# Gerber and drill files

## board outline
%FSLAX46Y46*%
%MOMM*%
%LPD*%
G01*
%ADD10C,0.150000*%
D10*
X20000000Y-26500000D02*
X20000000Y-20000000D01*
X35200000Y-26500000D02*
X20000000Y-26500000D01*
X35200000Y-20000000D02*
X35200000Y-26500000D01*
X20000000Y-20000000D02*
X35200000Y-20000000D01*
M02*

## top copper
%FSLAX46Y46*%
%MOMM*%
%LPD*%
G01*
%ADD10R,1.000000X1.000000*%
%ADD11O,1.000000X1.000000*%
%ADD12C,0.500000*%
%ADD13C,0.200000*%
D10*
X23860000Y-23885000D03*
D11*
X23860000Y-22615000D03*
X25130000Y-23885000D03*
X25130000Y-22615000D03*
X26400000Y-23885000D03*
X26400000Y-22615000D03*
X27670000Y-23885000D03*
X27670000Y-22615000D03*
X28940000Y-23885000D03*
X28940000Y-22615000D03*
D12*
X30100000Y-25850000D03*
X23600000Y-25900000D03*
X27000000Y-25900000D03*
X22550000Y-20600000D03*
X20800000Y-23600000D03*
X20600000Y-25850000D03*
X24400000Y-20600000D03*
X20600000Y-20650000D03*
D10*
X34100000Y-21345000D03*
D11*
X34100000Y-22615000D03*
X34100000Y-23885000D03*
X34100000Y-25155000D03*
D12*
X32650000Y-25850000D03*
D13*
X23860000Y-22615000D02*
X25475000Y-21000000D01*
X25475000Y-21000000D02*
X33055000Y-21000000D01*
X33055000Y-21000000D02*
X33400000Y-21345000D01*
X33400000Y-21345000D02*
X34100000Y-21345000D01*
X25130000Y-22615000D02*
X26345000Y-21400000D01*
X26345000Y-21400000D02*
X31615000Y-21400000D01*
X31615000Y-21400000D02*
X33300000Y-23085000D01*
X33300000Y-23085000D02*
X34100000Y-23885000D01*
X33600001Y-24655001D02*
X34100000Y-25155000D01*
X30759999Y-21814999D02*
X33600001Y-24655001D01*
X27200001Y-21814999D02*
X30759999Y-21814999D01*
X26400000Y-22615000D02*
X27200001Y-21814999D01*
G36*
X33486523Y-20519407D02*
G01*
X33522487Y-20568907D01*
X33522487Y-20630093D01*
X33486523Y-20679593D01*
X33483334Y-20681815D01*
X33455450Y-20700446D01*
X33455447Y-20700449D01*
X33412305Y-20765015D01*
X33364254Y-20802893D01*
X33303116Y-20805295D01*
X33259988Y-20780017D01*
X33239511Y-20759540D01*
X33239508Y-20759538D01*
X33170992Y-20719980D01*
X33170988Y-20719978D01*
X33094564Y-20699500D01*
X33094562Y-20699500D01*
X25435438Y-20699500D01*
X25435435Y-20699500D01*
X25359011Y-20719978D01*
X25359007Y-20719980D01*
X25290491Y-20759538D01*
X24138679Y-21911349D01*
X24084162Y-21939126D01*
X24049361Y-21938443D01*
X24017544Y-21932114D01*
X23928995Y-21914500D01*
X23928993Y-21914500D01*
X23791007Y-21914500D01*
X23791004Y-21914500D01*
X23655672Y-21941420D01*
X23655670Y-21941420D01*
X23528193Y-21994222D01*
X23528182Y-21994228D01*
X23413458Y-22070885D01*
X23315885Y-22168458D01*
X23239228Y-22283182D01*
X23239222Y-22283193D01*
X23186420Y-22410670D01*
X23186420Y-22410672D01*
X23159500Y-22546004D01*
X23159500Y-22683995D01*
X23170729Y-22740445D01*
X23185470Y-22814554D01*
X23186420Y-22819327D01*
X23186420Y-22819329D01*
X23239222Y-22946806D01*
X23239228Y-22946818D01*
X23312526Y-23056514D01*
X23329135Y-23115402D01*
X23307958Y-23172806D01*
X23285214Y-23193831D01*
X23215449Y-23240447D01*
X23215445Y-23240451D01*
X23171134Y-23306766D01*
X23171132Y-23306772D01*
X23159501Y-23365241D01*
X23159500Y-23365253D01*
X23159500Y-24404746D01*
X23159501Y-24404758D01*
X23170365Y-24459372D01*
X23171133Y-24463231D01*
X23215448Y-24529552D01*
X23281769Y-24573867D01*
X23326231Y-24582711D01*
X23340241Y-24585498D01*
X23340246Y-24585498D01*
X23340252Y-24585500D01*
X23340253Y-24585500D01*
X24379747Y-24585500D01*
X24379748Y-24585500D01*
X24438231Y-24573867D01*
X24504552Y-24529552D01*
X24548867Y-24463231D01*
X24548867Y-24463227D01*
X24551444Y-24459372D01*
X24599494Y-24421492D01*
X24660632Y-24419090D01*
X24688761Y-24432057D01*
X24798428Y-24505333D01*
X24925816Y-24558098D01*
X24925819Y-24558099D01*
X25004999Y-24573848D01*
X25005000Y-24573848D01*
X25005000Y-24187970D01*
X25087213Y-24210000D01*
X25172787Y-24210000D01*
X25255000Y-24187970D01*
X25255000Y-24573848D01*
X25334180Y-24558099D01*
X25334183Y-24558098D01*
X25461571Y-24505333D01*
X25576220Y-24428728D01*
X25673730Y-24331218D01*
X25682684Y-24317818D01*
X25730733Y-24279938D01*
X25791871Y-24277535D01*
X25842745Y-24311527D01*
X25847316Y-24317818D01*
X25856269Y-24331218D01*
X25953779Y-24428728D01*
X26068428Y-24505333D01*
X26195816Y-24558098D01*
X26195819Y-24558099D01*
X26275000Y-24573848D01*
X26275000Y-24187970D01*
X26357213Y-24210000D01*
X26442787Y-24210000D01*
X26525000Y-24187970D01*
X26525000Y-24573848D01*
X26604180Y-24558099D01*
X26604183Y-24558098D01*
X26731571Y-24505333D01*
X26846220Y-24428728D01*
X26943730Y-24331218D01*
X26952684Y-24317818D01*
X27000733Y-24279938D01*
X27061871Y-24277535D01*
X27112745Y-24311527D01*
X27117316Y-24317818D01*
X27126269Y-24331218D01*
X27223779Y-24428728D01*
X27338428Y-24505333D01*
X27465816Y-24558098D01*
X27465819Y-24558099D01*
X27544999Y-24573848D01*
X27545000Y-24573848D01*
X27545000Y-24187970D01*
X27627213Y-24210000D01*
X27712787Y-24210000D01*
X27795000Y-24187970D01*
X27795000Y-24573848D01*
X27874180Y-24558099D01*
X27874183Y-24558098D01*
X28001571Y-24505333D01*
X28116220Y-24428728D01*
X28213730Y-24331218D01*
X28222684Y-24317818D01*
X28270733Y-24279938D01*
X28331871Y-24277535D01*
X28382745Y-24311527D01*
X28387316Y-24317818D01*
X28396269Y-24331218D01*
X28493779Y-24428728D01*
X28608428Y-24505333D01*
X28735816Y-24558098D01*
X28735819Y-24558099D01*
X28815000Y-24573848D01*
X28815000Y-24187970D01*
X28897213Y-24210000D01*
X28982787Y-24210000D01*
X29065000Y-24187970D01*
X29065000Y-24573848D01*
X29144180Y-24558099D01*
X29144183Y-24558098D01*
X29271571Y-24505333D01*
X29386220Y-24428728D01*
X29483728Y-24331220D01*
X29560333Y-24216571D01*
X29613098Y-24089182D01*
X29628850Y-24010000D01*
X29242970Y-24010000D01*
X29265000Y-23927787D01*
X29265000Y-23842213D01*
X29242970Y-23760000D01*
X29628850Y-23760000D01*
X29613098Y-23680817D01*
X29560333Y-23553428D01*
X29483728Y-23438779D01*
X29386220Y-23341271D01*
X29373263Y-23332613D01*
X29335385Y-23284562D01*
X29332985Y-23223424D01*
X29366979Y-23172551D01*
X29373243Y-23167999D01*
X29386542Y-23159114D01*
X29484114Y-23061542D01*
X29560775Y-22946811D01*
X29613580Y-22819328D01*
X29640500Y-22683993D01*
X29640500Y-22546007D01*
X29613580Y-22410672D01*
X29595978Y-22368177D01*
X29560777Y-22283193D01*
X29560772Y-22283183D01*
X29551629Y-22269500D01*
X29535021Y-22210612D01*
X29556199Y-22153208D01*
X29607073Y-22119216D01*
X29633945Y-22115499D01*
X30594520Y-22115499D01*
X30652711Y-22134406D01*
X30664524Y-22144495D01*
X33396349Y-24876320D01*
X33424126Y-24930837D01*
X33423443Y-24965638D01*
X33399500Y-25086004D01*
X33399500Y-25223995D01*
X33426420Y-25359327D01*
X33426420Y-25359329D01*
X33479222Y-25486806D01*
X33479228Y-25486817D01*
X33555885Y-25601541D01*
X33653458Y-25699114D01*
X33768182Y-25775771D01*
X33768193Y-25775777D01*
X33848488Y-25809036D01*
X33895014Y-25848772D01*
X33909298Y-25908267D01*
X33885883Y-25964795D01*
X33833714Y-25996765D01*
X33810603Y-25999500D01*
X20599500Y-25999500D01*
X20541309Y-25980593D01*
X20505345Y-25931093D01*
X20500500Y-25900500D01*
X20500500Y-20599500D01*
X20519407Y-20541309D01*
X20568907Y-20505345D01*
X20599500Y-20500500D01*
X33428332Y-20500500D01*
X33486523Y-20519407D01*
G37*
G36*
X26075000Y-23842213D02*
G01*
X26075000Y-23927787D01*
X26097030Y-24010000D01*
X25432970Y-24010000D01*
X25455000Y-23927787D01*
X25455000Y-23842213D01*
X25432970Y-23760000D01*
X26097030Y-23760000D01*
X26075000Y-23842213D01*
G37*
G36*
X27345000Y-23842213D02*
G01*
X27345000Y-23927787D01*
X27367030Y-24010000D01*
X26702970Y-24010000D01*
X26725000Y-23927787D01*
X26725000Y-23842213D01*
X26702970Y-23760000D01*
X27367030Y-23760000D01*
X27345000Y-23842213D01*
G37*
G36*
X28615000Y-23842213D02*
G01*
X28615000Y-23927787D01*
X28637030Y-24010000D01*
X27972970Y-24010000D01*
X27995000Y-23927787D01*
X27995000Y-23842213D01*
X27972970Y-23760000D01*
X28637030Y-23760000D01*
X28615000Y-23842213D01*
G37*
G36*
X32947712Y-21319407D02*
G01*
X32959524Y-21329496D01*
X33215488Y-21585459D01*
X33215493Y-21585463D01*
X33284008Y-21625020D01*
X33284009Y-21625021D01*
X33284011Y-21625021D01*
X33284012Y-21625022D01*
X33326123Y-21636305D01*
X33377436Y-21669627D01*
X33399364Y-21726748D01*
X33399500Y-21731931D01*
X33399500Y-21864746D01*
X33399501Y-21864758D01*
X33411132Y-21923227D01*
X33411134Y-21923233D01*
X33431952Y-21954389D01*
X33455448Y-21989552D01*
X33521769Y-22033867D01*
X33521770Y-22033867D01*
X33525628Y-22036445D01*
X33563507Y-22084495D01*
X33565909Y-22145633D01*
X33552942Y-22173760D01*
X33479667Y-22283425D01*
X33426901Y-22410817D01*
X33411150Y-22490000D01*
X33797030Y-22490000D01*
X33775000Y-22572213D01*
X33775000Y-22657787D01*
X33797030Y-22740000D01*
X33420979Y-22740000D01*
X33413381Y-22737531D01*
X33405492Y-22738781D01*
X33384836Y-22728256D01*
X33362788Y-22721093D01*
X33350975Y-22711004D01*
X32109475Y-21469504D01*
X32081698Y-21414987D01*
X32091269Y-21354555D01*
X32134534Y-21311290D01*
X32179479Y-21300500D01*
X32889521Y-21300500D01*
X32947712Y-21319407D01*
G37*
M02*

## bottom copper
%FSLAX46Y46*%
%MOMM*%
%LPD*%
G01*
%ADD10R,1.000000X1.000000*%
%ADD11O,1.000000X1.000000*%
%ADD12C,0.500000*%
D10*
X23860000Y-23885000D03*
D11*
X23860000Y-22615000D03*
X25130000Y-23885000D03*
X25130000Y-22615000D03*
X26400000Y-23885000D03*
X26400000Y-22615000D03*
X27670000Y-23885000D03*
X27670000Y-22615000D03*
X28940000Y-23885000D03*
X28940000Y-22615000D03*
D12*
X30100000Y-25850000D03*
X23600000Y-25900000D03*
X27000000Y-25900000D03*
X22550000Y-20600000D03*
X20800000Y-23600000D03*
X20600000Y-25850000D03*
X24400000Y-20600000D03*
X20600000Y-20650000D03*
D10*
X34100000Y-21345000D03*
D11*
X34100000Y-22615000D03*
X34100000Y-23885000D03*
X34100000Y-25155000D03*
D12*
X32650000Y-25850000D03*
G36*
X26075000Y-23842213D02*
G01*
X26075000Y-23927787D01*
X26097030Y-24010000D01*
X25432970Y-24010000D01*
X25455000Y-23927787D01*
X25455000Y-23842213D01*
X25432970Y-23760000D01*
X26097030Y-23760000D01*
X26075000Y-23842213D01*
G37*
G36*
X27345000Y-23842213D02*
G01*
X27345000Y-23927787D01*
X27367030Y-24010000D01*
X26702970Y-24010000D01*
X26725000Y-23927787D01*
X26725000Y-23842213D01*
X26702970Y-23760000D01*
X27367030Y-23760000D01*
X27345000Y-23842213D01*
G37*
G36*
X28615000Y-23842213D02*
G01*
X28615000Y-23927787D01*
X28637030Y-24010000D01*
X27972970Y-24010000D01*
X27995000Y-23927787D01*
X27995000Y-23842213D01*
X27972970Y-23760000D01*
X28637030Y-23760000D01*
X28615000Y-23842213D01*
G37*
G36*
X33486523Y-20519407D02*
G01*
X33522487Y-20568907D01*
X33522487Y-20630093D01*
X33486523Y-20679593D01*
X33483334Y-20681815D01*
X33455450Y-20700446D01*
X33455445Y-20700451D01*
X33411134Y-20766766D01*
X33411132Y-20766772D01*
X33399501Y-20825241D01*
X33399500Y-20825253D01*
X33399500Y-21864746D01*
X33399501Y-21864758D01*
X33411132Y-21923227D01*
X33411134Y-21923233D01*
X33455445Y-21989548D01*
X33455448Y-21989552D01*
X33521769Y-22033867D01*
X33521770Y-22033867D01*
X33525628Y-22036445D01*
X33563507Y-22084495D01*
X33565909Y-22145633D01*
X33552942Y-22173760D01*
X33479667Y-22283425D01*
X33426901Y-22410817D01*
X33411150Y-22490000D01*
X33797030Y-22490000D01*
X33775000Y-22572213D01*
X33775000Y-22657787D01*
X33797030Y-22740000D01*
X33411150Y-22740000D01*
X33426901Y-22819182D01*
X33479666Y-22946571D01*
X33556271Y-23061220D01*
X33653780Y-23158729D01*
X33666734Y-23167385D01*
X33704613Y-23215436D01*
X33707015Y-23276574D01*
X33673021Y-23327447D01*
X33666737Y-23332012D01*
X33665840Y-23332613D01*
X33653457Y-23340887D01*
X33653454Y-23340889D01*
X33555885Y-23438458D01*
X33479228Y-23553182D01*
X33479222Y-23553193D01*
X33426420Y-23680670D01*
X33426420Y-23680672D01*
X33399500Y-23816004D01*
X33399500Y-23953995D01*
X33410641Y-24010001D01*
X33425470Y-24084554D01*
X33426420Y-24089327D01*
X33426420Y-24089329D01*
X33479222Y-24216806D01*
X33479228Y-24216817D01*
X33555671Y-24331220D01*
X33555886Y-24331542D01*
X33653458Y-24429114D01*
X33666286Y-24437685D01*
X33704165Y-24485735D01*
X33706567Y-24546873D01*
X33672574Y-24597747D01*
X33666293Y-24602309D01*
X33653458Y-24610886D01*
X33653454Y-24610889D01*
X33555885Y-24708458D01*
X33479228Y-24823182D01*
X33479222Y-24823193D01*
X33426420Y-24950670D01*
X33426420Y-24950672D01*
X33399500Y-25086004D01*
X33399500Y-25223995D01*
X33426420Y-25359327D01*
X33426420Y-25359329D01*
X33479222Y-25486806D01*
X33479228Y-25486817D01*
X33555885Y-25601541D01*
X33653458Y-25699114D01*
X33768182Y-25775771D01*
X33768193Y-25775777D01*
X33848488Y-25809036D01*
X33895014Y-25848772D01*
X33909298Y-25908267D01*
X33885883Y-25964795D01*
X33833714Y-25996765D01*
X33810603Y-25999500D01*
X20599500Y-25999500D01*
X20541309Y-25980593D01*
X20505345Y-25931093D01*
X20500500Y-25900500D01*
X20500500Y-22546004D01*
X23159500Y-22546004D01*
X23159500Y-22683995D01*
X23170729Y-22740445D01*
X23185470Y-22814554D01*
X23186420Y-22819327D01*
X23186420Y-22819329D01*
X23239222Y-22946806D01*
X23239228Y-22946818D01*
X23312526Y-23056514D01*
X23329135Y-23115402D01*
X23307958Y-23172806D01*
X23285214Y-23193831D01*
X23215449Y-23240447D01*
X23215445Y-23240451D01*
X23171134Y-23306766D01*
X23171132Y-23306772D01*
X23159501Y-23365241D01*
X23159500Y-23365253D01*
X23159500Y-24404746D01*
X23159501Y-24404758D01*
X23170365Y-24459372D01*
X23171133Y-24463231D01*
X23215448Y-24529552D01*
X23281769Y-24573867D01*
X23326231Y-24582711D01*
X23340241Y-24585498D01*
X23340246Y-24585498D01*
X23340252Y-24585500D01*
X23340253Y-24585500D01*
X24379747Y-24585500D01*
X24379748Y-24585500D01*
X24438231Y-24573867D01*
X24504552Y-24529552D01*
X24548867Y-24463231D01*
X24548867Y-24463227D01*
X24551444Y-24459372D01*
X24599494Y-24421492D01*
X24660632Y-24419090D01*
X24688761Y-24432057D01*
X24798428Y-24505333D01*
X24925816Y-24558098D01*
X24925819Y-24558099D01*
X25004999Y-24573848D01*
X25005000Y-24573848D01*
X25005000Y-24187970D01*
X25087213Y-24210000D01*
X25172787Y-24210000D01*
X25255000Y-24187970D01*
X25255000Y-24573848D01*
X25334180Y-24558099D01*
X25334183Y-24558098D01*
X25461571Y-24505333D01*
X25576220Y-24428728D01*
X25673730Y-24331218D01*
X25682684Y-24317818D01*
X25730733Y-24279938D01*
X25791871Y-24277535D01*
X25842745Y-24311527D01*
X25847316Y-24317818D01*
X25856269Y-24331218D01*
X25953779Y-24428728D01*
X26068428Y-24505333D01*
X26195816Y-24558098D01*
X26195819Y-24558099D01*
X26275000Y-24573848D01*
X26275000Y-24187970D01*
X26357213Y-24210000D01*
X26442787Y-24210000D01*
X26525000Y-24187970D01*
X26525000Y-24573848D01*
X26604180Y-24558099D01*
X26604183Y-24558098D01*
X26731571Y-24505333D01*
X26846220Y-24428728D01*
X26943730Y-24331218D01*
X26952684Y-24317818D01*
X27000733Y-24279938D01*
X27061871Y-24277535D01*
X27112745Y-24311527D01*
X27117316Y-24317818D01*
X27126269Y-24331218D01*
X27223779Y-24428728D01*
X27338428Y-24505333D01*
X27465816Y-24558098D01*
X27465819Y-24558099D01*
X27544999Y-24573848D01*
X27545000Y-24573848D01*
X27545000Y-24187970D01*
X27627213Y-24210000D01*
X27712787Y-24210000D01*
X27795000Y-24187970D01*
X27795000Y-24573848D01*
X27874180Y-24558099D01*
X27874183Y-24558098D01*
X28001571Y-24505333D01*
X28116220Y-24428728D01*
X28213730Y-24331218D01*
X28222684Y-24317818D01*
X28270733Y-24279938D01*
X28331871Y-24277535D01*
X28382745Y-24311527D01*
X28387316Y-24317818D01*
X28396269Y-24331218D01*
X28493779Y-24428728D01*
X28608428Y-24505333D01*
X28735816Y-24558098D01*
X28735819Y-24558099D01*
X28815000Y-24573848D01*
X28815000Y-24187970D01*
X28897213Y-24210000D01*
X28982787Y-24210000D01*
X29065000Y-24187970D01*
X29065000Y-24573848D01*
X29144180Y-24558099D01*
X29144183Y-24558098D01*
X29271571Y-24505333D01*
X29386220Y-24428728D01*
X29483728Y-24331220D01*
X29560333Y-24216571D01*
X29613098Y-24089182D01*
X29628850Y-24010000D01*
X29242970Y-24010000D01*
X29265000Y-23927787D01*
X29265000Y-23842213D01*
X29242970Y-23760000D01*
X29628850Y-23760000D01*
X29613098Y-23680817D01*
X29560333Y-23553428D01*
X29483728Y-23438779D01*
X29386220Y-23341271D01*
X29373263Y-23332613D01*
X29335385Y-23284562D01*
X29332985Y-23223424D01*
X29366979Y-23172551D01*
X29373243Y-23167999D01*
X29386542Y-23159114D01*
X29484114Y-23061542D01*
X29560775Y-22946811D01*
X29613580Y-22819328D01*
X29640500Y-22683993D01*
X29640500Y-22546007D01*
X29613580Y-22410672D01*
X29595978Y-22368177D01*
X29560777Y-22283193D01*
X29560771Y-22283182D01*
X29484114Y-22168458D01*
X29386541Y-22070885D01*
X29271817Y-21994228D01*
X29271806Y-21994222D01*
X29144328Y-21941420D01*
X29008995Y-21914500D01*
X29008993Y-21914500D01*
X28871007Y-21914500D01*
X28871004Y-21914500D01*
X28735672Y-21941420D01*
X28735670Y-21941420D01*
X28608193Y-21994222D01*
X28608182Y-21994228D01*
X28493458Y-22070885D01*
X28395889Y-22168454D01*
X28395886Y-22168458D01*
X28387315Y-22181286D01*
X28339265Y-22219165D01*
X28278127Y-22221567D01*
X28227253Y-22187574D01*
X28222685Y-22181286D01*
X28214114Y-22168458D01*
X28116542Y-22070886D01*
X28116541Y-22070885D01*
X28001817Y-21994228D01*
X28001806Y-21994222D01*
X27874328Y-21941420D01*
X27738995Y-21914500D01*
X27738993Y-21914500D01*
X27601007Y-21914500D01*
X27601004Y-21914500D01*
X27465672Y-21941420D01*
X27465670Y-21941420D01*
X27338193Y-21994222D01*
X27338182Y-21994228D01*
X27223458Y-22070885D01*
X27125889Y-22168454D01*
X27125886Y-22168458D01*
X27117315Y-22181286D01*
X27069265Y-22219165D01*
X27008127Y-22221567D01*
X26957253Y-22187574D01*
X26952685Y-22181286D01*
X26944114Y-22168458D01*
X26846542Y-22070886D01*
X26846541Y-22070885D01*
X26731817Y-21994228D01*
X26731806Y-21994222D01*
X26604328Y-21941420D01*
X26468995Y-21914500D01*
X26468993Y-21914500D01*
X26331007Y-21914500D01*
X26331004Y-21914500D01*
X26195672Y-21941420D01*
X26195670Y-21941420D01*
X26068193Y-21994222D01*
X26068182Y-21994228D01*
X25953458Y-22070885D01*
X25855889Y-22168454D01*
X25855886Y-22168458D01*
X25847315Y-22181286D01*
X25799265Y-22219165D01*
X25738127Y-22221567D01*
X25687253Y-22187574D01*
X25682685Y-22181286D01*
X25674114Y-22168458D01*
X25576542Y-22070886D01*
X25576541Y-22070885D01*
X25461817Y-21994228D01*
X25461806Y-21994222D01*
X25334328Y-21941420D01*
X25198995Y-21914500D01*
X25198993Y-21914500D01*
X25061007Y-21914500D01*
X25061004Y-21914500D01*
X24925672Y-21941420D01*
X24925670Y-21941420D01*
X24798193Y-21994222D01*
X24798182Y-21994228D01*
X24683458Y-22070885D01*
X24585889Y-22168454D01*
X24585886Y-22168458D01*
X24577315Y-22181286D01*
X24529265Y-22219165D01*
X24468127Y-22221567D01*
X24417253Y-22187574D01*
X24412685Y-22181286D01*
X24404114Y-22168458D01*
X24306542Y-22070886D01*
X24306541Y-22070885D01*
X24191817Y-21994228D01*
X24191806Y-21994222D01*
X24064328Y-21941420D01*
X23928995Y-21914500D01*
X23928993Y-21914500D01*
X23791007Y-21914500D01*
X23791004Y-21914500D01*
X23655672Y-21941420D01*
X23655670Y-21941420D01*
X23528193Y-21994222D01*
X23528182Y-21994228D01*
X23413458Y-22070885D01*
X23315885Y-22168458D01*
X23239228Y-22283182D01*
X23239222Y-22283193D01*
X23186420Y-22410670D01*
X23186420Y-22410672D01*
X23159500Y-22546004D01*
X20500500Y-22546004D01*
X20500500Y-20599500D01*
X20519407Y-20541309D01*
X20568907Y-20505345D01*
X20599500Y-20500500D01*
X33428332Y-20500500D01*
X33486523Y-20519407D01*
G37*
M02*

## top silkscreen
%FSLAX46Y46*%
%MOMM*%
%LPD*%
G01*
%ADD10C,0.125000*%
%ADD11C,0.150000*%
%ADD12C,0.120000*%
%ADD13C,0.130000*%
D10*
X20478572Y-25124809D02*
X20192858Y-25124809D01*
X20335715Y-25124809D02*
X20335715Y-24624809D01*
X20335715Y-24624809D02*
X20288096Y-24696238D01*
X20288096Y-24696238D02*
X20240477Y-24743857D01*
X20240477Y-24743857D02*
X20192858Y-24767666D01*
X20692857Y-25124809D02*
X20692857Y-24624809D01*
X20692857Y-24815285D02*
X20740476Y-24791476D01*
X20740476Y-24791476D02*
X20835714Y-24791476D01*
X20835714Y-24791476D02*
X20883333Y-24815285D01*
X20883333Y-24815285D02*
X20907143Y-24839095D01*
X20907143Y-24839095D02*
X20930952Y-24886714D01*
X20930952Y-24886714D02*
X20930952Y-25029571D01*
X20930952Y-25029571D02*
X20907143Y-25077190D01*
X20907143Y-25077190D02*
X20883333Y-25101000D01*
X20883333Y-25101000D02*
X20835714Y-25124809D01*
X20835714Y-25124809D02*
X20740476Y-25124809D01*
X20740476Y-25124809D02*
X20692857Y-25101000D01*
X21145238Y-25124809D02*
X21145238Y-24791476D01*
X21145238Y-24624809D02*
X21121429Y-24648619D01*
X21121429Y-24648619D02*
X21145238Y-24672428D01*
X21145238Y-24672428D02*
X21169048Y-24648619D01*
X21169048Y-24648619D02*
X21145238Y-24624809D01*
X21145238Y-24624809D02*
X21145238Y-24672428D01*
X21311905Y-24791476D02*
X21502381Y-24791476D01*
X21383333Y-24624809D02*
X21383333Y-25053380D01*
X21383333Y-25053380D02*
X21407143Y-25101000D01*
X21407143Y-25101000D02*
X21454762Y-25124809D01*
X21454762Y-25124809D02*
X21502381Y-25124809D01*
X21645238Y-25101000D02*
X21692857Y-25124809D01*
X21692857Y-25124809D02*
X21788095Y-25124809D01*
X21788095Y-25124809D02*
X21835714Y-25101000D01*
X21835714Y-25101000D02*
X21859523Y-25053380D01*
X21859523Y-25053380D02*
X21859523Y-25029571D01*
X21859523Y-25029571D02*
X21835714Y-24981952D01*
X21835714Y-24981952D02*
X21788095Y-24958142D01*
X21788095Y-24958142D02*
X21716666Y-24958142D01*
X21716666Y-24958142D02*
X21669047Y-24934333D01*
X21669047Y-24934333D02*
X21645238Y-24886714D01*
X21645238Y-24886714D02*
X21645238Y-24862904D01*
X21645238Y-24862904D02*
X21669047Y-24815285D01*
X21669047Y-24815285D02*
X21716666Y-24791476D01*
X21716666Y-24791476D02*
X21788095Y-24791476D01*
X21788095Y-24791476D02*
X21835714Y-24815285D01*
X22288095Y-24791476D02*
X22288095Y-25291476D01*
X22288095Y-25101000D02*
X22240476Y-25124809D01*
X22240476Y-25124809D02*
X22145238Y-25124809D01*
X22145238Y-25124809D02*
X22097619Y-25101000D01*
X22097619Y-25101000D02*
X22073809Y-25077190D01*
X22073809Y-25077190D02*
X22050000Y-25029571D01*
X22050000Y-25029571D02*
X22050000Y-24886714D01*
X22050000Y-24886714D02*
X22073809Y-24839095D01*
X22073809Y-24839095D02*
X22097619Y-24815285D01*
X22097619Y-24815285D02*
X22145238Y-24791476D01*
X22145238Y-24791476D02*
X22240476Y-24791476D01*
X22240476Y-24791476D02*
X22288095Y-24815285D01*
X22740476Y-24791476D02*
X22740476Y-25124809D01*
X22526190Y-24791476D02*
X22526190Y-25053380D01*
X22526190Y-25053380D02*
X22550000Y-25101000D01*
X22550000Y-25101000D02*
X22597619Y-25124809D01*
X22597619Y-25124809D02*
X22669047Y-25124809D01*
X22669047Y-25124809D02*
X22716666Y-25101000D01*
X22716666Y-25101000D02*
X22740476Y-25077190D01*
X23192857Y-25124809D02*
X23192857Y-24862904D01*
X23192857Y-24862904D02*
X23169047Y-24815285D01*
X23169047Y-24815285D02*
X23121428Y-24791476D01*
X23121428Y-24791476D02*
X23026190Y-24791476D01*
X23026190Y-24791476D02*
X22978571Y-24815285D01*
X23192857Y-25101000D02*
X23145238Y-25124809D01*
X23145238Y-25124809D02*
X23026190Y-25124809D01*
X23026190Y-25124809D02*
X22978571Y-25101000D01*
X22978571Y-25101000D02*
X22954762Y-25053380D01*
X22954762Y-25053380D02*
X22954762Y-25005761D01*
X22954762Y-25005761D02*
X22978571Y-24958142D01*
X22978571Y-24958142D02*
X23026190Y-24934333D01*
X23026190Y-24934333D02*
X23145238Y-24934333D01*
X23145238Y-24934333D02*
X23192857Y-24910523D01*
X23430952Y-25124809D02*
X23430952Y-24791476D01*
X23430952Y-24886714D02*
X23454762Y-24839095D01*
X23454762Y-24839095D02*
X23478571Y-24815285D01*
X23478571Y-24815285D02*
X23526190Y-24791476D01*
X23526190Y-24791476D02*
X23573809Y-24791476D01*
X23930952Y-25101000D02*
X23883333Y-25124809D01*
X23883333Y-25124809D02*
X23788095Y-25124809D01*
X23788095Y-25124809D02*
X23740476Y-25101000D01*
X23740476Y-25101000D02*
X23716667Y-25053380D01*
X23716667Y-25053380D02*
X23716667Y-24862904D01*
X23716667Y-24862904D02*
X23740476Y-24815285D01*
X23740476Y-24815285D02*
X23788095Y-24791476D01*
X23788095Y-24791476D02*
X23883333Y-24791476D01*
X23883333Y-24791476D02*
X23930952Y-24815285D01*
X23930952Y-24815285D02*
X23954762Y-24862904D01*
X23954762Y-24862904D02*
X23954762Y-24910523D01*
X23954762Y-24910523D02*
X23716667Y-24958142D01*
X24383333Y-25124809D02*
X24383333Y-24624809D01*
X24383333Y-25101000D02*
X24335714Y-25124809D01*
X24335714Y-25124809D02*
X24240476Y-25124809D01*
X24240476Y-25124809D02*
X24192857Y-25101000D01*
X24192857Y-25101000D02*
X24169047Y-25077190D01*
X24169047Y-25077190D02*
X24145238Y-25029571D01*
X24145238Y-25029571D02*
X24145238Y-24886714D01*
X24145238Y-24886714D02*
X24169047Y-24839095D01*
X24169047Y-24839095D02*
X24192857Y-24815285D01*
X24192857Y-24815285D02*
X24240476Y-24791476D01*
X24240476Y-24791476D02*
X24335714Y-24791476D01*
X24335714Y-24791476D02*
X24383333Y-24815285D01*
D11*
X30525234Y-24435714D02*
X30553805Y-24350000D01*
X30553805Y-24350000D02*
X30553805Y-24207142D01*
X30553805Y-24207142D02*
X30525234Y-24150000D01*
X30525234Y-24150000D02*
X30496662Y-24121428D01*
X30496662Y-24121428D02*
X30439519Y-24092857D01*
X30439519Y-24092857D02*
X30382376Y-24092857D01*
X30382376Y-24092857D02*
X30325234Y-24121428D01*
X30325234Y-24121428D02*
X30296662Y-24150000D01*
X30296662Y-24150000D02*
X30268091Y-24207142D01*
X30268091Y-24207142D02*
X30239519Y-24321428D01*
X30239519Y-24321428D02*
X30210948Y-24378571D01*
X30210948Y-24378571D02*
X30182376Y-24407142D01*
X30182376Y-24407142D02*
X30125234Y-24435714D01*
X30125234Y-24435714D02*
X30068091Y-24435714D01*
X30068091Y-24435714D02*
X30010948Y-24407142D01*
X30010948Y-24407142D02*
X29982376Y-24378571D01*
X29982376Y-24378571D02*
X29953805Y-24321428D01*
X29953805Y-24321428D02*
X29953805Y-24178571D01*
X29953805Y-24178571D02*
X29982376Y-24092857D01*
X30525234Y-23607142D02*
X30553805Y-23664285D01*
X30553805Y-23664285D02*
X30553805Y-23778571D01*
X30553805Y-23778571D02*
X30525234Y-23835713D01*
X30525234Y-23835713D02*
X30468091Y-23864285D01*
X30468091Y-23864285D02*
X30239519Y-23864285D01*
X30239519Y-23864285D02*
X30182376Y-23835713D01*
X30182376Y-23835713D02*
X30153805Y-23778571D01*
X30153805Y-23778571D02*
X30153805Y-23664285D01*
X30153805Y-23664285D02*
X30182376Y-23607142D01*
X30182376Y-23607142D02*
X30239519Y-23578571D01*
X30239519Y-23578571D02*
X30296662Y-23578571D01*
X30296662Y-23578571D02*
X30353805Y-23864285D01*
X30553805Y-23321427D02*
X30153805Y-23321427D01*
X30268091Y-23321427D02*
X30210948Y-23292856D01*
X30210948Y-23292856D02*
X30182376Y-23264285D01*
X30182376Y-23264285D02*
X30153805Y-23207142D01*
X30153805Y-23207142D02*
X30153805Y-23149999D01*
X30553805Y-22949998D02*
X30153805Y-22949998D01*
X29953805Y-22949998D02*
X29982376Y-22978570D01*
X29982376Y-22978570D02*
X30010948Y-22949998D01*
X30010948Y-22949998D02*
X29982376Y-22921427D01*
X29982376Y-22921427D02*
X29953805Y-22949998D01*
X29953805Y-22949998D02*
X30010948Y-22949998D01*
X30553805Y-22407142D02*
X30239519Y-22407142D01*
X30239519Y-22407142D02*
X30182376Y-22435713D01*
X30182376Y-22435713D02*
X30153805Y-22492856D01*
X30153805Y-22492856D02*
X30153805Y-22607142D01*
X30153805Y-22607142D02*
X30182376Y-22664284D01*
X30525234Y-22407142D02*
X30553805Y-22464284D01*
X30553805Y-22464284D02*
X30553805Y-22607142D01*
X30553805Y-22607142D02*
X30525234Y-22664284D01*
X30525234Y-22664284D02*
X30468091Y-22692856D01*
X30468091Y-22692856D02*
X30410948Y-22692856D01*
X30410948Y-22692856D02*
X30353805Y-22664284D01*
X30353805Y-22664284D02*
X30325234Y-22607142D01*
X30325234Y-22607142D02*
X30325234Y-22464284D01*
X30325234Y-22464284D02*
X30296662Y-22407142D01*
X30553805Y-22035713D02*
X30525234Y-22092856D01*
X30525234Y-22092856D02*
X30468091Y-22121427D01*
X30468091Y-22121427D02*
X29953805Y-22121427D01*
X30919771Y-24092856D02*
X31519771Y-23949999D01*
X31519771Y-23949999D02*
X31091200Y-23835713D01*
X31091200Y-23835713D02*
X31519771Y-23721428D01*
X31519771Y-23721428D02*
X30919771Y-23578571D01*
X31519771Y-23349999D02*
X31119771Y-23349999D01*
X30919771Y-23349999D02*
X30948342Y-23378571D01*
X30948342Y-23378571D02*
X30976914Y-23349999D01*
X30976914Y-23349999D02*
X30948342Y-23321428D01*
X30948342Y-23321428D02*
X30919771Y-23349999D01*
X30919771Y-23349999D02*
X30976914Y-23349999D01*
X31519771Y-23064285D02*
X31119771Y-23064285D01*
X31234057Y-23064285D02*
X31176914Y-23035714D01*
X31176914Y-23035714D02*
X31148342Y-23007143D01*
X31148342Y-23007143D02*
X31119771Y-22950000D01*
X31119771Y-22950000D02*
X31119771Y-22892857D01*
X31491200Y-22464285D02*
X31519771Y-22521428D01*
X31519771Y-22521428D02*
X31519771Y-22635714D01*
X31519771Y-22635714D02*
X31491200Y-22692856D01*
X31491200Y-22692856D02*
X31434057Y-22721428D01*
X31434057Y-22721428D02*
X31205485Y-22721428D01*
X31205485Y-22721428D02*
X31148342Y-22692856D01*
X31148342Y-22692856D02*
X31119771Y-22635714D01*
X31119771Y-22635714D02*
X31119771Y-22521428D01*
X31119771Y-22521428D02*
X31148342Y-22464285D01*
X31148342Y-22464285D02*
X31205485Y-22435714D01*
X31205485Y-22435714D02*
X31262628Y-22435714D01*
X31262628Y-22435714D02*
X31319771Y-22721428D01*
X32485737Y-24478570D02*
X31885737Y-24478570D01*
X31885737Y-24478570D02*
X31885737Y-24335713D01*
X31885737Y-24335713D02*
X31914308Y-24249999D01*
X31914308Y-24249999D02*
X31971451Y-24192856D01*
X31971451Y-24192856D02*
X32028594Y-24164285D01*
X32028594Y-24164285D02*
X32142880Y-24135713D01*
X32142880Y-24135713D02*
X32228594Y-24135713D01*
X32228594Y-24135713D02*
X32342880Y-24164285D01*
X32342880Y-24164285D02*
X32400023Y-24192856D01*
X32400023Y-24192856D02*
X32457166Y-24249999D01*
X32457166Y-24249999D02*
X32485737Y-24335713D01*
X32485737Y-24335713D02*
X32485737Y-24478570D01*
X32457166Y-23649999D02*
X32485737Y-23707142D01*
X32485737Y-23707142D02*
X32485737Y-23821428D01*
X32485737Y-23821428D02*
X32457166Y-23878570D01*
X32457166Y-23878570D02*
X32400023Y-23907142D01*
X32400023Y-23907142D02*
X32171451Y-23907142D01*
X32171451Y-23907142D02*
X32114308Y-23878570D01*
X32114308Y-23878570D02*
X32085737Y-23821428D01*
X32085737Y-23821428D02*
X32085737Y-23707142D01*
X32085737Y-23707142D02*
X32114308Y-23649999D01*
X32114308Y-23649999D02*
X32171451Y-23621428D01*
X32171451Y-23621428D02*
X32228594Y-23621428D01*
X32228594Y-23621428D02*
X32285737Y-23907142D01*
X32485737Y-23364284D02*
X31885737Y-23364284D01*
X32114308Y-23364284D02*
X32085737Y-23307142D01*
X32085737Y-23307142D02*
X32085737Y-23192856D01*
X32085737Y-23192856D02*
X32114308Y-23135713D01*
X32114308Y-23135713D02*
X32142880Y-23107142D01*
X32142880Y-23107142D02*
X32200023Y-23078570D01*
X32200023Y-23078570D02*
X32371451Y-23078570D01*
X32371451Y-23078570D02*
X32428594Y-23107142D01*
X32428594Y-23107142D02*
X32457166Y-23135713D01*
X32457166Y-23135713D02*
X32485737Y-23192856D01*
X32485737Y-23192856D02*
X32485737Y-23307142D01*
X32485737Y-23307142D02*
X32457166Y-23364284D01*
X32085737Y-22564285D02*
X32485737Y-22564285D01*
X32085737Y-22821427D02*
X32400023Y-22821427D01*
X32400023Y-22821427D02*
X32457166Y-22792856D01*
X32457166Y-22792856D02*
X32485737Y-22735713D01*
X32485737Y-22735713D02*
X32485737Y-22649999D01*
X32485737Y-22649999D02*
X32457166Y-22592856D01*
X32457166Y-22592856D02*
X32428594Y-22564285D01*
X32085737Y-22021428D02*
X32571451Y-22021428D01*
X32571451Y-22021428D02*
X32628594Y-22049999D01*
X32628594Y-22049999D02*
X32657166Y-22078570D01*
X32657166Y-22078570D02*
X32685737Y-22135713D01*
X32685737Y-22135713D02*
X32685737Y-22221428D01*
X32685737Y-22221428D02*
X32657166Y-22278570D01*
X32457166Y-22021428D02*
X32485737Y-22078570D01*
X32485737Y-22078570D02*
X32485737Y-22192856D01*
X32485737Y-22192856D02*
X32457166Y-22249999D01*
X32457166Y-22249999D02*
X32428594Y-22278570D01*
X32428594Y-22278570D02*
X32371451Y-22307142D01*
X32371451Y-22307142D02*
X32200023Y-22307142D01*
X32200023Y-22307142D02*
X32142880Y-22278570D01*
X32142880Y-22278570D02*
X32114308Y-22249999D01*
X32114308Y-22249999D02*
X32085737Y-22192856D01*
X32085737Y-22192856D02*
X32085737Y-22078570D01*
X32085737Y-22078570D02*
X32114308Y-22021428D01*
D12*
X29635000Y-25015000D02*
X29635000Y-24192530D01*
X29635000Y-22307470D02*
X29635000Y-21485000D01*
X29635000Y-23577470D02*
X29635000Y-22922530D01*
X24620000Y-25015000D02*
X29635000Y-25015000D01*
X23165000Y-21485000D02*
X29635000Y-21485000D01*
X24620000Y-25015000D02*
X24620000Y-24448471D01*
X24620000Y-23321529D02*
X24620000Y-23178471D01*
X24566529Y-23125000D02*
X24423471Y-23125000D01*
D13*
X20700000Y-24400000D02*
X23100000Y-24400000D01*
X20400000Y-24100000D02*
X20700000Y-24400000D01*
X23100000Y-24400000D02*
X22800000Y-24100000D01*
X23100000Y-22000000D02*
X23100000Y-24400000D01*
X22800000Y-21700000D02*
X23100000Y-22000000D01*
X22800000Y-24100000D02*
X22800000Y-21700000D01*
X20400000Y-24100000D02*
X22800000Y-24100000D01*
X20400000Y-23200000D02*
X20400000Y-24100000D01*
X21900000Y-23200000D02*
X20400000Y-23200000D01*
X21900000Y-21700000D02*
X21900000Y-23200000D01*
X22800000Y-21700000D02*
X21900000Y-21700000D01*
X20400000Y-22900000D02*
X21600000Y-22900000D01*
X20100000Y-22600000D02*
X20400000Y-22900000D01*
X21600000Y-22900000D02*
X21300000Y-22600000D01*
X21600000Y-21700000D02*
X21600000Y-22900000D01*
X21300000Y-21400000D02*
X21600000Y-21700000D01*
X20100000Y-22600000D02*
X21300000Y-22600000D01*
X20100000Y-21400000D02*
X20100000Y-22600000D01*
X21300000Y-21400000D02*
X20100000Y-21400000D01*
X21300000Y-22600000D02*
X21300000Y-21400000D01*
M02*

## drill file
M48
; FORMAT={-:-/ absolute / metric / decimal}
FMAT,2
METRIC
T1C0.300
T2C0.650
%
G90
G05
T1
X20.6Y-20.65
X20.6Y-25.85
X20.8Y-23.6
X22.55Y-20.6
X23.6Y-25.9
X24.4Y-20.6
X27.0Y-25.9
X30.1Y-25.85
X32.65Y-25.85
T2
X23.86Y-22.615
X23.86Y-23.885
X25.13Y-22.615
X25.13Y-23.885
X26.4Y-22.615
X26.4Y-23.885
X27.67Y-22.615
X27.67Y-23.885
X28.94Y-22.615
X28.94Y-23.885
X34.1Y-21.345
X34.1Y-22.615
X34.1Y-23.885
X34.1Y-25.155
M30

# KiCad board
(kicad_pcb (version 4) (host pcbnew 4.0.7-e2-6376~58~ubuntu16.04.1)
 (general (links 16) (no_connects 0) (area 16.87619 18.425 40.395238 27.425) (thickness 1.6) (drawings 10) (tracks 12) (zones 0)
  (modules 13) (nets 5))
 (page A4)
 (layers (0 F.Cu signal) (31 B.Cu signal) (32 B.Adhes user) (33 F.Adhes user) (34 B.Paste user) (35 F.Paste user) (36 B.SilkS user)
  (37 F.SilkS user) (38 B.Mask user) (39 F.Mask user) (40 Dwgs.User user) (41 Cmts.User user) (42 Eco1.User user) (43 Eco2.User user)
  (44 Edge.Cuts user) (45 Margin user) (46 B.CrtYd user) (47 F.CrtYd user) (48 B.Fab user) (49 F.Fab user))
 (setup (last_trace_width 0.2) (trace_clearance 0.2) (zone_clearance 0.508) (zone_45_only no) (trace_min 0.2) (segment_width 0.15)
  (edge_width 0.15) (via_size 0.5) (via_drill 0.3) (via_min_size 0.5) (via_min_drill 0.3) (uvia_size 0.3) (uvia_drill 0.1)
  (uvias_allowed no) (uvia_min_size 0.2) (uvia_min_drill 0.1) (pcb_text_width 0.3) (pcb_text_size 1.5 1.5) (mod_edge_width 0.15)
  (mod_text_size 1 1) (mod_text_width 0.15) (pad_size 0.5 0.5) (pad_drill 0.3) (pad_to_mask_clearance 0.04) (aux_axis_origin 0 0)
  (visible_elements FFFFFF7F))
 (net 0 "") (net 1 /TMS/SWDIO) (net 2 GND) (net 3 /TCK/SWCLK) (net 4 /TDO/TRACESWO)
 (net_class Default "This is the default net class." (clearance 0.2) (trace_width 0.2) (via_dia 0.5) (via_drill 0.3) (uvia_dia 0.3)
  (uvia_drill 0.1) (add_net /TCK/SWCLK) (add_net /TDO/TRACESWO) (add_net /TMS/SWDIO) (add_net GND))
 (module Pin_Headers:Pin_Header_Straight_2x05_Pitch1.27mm (layer F.Cu) (at 26.4 23.25 90)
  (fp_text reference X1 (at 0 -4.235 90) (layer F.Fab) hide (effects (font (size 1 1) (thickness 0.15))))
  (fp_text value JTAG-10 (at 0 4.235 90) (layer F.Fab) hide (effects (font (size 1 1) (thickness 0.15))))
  (fp_line (start -1.765 3.235) (end -0.94253 3.235) (layer F.SilkS) (width 0.12))
  (fp_line (start 0.94253 3.235) (end 1.765 3.235) (layer F.SilkS) (width 0.12))
  (fp_line (start -0.32747 3.235) (end 0.32747 3.235) (layer F.SilkS) (width 0.12))
  (fp_line (start -1.765 -1.78) (end -1.765 3.235) (layer F.SilkS) (width 0.12))
  (fp_line (start 1.765 -3.235) (end 1.765 3.235) (layer F.SilkS) (width 0.12))
  (fp_line (start -1.765 -1.78) (end -1.198471 -1.78) (layer F.SilkS) (width 0.12))
  (fp_line (start -0.071529 -1.78) (end 0.071529 -1.78) (layer F.SilkS) (width 0.12))
  (fp_line (start 0.125 -1.833471) (end 0.125 -1.976529) (layer F.SilkS) (width 0.12))
  (pad 1 thru_hole rect (at -0.635 -2.54 90) (size 1 1) (drill 0.65) (layers *.Cu *.Mask))
  (pad 2 thru_hole oval (at 0.635 -2.54 90) (size 1 1) (drill 0.65) (layers *.Cu *.Mask) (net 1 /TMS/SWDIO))
  (pad 3 thru_hole oval (at -0.635 -1.27 90) (size 1 1) (drill 0.65) (layers *.Cu *.Mask) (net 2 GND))
  (pad 4 thru_hole oval (at 0.635 -1.27 90) (size 1 1) (drill 0.65) (layers *.Cu *.Mask) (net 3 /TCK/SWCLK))
  (pad 5 thru_hole oval (at -0.635 0 90) (size 1 1) (drill 0.65) (layers *.Cu *.Mask) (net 2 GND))
  (pad 6 thru_hole oval (at 0.635 0 90) (size 1 1) (drill 0.65) (layers *.Cu *.Mask) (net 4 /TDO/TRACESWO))
  (pad 7 thru_hole oval (at -0.635 1.27 90) (size 1 1) (drill 0.65) (layers *.Cu *.Mask) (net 2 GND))
  (pad 8 thru_hole oval (at 0.635 1.27 90) (size 1 1) (drill 0.65) (layers *.Cu *.Mask))
  (pad 9 thru_hole oval (at -0.635 2.54 90) (size 1 1) (drill 0.65) (layers *.Cu *.Mask) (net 2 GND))
  (pad 10 thru_hole oval (at 0.635 2.54 90) (size 1 1) (drill 0.65) (layers *.Cu *.Mask)))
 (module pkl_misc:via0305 (layer F.Cu) (at 30.1 25.85)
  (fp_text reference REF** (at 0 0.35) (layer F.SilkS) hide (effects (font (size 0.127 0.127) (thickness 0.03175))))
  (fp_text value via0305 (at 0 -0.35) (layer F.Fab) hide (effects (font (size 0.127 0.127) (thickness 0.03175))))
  (pad 1 thru_hole circle (at 0 0) (size 0.5 0.5) (drill 0.3) (layers *.Cu) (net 2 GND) (zone_connect 2)))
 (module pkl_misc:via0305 (layer F.Cu) (at 23.6 25.9)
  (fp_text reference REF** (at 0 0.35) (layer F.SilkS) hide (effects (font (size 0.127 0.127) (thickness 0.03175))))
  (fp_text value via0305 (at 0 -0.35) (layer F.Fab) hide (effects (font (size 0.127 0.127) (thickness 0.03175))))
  (pad 1 thru_hole circle (at 0 0) (size 0.5 0.5) (drill 0.3) (layers *.Cu) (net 2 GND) (zone_connect 2)))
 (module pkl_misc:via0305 (layer F.Cu) (at 27 25.9)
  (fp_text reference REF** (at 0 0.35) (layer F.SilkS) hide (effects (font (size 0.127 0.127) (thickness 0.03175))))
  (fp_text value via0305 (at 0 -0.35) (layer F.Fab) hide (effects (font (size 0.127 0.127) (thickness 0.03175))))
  (pad 1 thru_hole circle (at 0 0) (size 0.5 0.5) (drill 0.3) (layers *.Cu) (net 2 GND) (zone_connect 2)))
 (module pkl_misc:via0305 (layer F.Cu) (at 22.55 20.6)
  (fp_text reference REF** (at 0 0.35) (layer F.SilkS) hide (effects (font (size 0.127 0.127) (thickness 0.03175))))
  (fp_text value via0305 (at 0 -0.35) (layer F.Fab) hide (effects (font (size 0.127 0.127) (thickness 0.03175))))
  (pad 1 thru_hole circle (at 0 0) (size 0.5 0.5) (drill 0.3) (layers *.Cu) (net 2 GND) (zone_connect 2)))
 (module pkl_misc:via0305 (layer F.Cu) (at 20.8 23.6)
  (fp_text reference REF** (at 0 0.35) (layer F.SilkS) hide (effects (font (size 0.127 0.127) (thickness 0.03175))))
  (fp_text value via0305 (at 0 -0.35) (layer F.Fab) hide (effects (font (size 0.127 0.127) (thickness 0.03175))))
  (pad 1 thru_hole circle (at 0 0) (size 0.5 0.5) (drill 0.3) (layers *.Cu) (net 2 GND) (zone_connect 2)))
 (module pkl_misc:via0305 (layer F.Cu) (at 20.6 25.85)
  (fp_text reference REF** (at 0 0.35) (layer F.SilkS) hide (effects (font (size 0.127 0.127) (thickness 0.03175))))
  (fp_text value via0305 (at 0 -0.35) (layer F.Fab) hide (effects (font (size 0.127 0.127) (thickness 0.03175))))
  (pad 1 thru_hole circle (at 0 0) (size 0.5 0.5) (drill 0.3) (layers *.Cu) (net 2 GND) (zone_connect 2)))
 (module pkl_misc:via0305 (layer F.Cu) (at 24.4 20.6)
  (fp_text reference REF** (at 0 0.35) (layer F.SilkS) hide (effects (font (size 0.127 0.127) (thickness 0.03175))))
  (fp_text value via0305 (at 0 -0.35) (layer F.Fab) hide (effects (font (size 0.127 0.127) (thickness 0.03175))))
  (pad 1 thru_hole circle (at 0 0) (size 0.5 0.5) (drill 0.3) (layers *.Cu) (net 2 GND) (zone_connect 2)))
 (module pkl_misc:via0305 (layer F.Cu) (at 20.6 20.65)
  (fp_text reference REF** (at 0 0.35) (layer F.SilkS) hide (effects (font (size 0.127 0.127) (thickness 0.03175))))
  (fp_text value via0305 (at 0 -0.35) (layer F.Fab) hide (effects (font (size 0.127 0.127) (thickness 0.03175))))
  (pad 1 thru_hole circle (at 0 0) (size 0.5 0.5) (drill 0.3) (layers *.Cu) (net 2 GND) (zone_connect 2)))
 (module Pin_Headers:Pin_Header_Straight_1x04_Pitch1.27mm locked (layer B.Cu) (at 34.1 23.25 180)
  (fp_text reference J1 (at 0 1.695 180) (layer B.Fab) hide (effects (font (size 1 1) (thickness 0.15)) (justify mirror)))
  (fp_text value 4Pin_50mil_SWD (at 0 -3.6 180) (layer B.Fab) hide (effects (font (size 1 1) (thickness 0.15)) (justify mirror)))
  (pad 1 thru_hole rect (at 0 1.905 180) (size 1 1) (drill 0.65) (layers *.Cu *.Mask) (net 1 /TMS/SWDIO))
  (pad 2 thru_hole oval (at 0 0.635 180) (size 1 1) (drill 0.65) (layers *.Cu *.Mask) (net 2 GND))
  (pad 3 thru_hole oval (at 0 -0.635 180) (size 1 1) (drill 0.65) (layers *.Cu *.Mask) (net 3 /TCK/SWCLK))
  (pad 4 thru_hole oval (at 0 -1.905 180) (size 1 1) (drill 0.65) (layers *.Cu *.Mask) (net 4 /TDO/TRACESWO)))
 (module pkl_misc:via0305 (layer F.Cu) (at 32.65 25.85)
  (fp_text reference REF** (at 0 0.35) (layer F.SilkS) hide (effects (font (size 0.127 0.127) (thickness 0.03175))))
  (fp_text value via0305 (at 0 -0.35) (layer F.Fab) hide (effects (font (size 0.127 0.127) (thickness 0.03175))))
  (pad 1 thru_hole circle (at 0 0) (size 0.5 0.5) (drill 0.3) (layers *.Cu) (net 2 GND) (zone_connect 2)))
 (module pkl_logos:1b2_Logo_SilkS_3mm (layer B.Cu) (at 21.6 22.9 180)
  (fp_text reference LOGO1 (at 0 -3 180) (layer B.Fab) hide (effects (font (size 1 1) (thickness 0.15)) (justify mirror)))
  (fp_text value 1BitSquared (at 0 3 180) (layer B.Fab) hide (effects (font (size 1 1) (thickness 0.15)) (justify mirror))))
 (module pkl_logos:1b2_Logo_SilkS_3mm (layer F.Cu) (at 21.6 22.9)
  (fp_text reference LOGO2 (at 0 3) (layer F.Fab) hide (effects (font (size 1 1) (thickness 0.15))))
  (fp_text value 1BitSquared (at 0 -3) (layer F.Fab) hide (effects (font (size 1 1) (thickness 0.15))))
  (fp_line (start -0.9 1.5) (end 1.5 1.5) (layer F.SilkS) (width 0.13))
  (fp_line (start -1.2 1.2) (end -0.9 1.5) (layer F.SilkS) (width 0.13))
  (fp_line (start 1.5 1.5) (end 1.2 1.2) (layer F.SilkS) (width 0.13))
  (fp_line (start 1.5 -0.9) (end 1.5 1.5) (layer F.SilkS) (width 0.13))
  (fp_line (start 1.2 -1.2) (end 1.5 -0.9) (layer F.SilkS) (width 0.13))
  (fp_line (start 1.2 1.2) (end 1.2 -1.2) (layer F.SilkS) (width 0.13))
  (fp_line (start -1.2 1.2) (end 1.2 1.2) (layer F.SilkS) (width 0.13))
  (fp_line (start -1.2 0.3) (end -1.2 1.2) (layer F.SilkS) (width 0.13))
  (fp_line (start 0.3 0.3) (end -1.2 0.3) (layer F.SilkS) (width 0.13))
  (fp_line (start 0.3 -1.2) (end 0.3 0.3) (layer F.SilkS) (width 0.13))
  (fp_line (start 1.2 -1.2) (end 0.3 -1.2) (layer F.SilkS) (width 0.13))
  (fp_line (start -1.2 0) (end 0 0) (layer F.SilkS) (width 0.13))
  (fp_line (start -1.5 -0.3) (end -1.2 0) (layer F.SilkS) (width 0.13))
  (fp_line (start 0 0) (end -0.3 -0.3) (layer F.SilkS) (width 0.13))
  (fp_line (start 0 -1.2) (end 0 0) (layer F.SilkS) (width 0.13))
  (fp_line (start -0.3 -1.5) (end 0 -1.2) (layer F.SilkS) (width 0.13))
  (fp_line (start -1.5 -0.3) (end -0.3 -0.3) (layer F.SilkS) (width 0.13))
  (fp_line (start -1.5 -1.5) (end -1.5 -0.3) (layer F.SilkS) (width 0.13))
  (fp_line (start -0.3 -1.5) (end -1.5 -1.5) (layer F.SilkS) (width 0.13))
  (fp_line (start -0.3 -0.3) (end -0.3 -1.5) (layer F.SilkS) (width 0.13)))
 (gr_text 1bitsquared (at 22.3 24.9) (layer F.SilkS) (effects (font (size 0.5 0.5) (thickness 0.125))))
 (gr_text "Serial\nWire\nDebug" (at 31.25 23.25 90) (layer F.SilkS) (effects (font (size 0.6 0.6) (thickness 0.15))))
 (gr_line (start 20 26.5) (end 20 20) (layer Edge.Cuts) (width 0.15))
 (gr_line (start 35.2 26.5) (end 20 26.5) (layer Edge.Cuts) (width 0.15))
 (gr_line (start 35.2 20) (end 35.2 26.5) (layer Edge.Cuts) (width 0.15))
 (gr_line (start 20 20) (end 35.2 20) (layer Edge.Cuts) (width 0.15))
 (segment (start 23.86 22.615) (end 25.475 21) (width 0.2) (layer F.Cu) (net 1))
 (segment (start 25.475 21) (end 33.055 21) (width 0.2) (layer F.Cu) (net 1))
 (segment (start 33.055 21) (end 33.4 21.345) (width 0.2) (layer F.Cu) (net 1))
 (segment (start 33.4 21.345) (end 34.1 21.345) (width 0.2) (layer F.Cu) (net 1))
 (segment (start 25.13 22.615) (end 26.345 21.4) (width 0.2) (layer F.Cu) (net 3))
 (segment (start 26.345 21.4) (end 31.615 21.4) (width 0.2) (layer F.Cu) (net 3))
 (segment (start 31.615 21.4) (end 33.3 23.085) (width 0.2) (layer F.Cu) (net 3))
 (segment (start 33.3 23.085) (end 34.1 23.885) (width 0.2) (layer F.Cu) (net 3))
 (segment (start 33.600001 24.655001) (end 34.1 25.155) (width 0.2) (layer F.Cu) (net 4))
 (segment (start 30.759999 21.814999) (end 33.600001 24.655001) (width 0.2) (layer F.Cu) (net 4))
 (segment (start 27.200001 21.814999) (end 30.759999 21.814999) (width 0.2) (layer F.Cu) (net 4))
 (segment (start 26.4 22.615) (end 27.200001 21.814999) (width 0.2) (layer F.Cu) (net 4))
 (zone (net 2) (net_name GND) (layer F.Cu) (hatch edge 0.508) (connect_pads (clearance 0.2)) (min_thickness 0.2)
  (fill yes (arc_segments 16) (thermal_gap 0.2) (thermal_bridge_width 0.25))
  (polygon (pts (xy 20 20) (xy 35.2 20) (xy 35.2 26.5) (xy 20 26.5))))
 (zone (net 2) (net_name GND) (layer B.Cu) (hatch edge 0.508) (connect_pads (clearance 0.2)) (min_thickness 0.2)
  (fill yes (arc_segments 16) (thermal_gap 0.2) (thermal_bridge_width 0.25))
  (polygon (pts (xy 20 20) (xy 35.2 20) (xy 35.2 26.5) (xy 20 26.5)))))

